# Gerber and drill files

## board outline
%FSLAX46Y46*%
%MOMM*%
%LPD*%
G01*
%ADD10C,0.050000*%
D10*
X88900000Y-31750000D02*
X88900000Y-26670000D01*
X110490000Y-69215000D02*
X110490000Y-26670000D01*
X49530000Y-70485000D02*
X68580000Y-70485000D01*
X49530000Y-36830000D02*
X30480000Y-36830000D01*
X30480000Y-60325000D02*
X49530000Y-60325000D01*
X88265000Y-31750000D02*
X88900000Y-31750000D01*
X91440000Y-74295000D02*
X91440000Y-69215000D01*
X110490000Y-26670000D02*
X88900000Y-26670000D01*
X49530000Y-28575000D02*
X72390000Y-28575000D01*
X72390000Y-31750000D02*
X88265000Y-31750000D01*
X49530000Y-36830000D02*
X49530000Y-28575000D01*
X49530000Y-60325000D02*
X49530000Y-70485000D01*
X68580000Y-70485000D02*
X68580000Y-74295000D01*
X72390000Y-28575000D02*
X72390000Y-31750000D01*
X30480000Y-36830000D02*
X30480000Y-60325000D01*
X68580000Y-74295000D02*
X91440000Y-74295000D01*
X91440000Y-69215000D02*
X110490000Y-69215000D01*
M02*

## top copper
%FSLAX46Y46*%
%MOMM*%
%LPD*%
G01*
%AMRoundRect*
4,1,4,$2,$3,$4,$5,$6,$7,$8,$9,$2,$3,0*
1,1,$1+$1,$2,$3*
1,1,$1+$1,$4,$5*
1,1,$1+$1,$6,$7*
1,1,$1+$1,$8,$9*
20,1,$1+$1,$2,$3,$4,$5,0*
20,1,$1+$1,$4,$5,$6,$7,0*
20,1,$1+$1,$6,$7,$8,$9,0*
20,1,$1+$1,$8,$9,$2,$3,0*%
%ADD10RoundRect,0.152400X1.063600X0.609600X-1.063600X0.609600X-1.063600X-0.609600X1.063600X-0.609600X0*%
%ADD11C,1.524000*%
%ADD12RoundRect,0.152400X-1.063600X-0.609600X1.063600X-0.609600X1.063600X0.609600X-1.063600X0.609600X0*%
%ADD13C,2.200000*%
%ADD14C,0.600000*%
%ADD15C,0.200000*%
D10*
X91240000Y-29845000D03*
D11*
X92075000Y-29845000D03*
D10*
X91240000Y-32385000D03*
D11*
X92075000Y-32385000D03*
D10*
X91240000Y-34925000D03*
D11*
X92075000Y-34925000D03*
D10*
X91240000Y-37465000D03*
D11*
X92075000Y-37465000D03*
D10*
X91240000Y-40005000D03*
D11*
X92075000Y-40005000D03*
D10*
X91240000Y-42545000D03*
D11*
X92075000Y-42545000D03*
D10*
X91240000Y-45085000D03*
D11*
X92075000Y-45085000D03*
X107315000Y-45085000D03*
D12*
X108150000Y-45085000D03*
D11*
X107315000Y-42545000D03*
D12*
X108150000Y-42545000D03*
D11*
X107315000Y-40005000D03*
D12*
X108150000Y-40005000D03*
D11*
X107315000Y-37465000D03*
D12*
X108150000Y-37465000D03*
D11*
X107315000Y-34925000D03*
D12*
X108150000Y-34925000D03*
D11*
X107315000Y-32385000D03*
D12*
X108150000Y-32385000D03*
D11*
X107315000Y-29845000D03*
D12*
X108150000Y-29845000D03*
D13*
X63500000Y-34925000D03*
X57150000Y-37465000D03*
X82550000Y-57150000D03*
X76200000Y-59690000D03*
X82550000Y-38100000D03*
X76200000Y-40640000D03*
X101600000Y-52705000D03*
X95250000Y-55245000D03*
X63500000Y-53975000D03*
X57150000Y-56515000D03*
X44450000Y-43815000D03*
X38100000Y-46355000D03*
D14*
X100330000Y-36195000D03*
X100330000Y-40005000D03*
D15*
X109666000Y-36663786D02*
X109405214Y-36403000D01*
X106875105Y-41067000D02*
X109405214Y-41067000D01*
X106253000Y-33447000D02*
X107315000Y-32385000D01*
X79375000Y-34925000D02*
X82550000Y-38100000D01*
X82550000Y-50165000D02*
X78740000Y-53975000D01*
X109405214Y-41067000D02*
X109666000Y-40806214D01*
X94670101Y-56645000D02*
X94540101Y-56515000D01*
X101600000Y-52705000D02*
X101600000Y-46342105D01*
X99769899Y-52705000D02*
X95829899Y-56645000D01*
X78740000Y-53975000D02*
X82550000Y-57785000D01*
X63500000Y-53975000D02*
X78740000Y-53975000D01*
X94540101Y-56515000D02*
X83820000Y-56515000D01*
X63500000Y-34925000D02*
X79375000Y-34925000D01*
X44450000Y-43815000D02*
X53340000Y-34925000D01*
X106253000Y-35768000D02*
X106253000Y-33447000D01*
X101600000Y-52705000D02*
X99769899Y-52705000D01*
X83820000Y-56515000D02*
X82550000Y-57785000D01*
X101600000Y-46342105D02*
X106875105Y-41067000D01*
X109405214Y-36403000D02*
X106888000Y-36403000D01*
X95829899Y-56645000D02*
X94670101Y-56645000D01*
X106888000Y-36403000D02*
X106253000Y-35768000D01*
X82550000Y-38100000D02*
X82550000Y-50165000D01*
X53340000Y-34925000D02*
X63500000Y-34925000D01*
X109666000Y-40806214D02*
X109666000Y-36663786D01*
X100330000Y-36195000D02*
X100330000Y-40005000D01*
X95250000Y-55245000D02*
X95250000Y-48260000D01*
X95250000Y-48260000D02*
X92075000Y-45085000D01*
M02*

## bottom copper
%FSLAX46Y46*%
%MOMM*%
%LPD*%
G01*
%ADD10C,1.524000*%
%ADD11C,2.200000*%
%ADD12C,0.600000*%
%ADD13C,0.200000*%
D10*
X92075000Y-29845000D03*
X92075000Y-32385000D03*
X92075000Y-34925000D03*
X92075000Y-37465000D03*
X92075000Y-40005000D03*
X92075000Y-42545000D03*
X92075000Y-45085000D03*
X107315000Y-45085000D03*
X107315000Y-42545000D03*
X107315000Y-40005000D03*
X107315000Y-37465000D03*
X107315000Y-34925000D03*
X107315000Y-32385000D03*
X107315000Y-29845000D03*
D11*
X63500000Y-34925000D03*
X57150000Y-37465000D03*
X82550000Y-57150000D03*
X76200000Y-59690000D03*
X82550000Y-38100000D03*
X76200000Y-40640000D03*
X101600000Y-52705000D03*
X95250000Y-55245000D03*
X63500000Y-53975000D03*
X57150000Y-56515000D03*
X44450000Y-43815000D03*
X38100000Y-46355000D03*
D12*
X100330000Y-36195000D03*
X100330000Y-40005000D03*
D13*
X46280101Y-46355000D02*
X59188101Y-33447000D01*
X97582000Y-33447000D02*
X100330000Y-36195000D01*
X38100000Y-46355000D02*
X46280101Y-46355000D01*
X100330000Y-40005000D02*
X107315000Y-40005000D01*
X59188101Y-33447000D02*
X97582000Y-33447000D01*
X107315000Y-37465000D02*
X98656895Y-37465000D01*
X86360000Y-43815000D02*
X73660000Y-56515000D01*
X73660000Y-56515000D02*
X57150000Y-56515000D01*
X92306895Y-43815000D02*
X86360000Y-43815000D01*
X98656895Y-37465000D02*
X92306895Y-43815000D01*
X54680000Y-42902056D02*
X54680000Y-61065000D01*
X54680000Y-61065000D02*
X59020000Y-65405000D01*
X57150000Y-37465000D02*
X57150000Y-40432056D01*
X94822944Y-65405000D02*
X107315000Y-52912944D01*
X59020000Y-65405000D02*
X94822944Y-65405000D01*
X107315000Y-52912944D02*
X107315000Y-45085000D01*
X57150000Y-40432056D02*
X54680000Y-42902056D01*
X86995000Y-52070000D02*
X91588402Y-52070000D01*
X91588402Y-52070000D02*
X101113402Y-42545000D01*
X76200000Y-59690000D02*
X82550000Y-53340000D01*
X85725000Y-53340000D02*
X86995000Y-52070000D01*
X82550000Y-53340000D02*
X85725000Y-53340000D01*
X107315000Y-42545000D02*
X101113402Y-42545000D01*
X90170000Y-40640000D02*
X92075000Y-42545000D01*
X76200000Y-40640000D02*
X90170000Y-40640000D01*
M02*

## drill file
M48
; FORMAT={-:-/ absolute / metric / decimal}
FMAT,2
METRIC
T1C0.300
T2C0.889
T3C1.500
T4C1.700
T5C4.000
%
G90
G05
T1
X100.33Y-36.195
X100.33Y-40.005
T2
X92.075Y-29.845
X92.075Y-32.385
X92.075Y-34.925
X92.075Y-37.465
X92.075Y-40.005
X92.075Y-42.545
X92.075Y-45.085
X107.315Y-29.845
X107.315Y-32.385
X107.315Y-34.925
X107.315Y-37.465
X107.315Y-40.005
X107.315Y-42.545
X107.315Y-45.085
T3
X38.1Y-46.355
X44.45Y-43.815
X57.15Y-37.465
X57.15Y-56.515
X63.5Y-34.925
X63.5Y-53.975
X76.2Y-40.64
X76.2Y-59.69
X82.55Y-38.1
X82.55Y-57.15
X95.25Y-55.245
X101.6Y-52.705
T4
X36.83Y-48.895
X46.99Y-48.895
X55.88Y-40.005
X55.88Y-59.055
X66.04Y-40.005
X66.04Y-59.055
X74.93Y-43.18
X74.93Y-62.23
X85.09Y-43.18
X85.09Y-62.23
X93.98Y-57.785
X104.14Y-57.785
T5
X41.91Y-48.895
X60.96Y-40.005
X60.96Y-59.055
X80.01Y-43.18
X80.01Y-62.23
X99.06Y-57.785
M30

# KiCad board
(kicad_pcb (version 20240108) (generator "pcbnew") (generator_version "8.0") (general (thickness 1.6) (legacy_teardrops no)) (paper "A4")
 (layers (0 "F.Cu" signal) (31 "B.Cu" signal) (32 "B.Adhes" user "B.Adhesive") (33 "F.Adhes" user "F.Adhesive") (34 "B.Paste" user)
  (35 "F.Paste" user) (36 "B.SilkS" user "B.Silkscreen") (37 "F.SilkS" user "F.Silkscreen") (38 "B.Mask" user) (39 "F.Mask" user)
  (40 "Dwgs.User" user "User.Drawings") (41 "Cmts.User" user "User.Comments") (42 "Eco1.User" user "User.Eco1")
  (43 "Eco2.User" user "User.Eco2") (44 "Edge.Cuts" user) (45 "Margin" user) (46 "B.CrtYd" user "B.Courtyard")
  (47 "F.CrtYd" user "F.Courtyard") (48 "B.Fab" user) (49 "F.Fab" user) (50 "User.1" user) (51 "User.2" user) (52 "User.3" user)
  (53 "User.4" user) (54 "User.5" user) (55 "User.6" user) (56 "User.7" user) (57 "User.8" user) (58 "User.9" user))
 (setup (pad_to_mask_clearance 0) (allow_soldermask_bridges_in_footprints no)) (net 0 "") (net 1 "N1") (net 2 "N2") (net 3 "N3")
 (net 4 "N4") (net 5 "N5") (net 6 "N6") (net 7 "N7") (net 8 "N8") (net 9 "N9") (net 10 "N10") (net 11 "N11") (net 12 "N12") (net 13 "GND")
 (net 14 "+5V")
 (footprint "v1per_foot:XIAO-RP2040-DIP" (layer "F.Cu") (at 99.695 37.465)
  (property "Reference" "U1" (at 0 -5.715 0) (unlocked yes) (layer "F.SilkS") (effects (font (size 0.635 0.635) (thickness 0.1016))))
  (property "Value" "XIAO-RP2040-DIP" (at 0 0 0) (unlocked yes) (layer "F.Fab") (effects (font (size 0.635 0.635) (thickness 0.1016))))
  (pad "1" smd roundrect (at -8.455 -7.62 180) (size 2.432 1.524) (layers "F.Cu" "F.Mask") (roundrect_rratio 0.1) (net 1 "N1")
   (thermal_bridge_angle 45))
  (pad "1" thru_hole circle (at -7.62 -7.62 180) (size 1.524 1.524) (drill 0.889) (layers "*.Cu" "*.Mask") (remove_unused_layers no)
   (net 1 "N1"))
  (pad "2" smd roundrect (at -8.455 -5.08 180) (size 2.432 1.524) (layers "F.Cu" "F.Mask") (roundrect_rratio 0.1) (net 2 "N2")
   (thermal_bridge_angle 45))
  (pad "2" thru_hole circle (at -7.62 -5.08 180) (size 1.524 1.524) (drill 0.889) (layers "*.Cu" "*.Mask") (remove_unused_layers no)
   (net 2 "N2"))
  (pad "3" smd roundrect (at -8.455 -2.54 180) (size 2.432 1.524) (layers "F.Cu" "F.Mask") (roundrect_rratio 0.1) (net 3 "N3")
   (thermal_bridge_angle 45))
  (pad "3" thru_hole circle (at -7.62 -2.54 180) (size 1.524 1.524) (drill 0.889) (layers "*.Cu" "*.Mask") (remove_unused_layers no)
   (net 3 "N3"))
  (pad "4" smd roundrect (at -8.455 0 180) (size 2.432 1.524) (layers "F.Cu" "F.Mask") (roundrect_rratio 0.1) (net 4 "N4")
   (thermal_bridge_angle 45))
  (pad "4" thru_hole circle (at -7.62 0 180) (size 1.524 1.524) (drill 0.889) (layers "*.Cu" "*.Mask") (remove_unused_layers no)
   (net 4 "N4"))
  (pad "5" smd roundrect (at -8.455 2.54 180) (size 2.432 1.524) (layers "F.Cu" "F.Mask") (roundrect_rratio 0.1) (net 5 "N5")
   (thermal_bridge_angle 45))
  (pad "5" thru_hole circle (at -7.62 2.54 180) (size 1.524 1.524) (drill 0.889) (layers "*.Cu" "*.Mask") (remove_unused_layers no)
   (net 5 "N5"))
  (pad "6" smd roundrect (at -8.455 5.08 180) (size 2.432 1.524) (layers "F.Cu" "F.Mask") (roundrect_rratio 0.1) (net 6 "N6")
   (thermal_bridge_angle 45))
  (pad "6" thru_hole circle (at -7.62 5.08 180) (size 1.524 1.524) (drill 0.889) (layers "*.Cu" "*.Mask") (remove_unused_layers no)
   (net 6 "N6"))
  (pad "7" smd roundrect (at -8.455 7.62 180) (size 2.432 1.524) (layers "F.Cu" "F.Mask") (roundrect_rratio 0.1) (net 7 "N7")
   (thermal_bridge_angle 45))
  (pad "7" thru_hole circle (at -7.62 7.62 180) (size 1.524 1.524) (drill 0.889) (layers "*.Cu" "*.Mask") (remove_unused_layers no)
   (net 7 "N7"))
  (pad "8" thru_hole circle (at 7.62 7.62) (size 1.524 1.524) (drill 0.889) (layers "*.Cu" "*.Mask") (remove_unused_layers no) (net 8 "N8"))
  (pad "8" smd roundrect (at 8.455 7.62) (size 2.432 1.524) (layers "F.Cu" "F.Mask") (roundrect_rratio 0.1) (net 8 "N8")
   (thermal_bridge_angle 45))
  (pad "9" thru_hole circle (at 7.62 5.08) (size 1.524 1.524) (drill 0.889) (layers "*.Cu" "*.Mask") (remove_unused_layers no) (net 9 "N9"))
  (pad "9" smd roundrect (at 8.455 5.08) (size 2.432 1.524) (layers "F.Cu" "F.Mask") (roundrect_rratio 0.1) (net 9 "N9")
   (thermal_bridge_angle 45))
  (pad "10" thru_hole circle (at 7.62 2.54) (size 1.524 1.524) (drill 0.889) (layers "*.Cu" "*.Mask") (remove_unused_layers no)
   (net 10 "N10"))
  (pad "10" smd roundrect (at 8.455 2.54) (size 2.432 1.524) (layers "F.Cu" "F.Mask") (roundrect_rratio 0.1) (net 10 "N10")
   (thermal_bridge_angle 45))
  (pad "11" thru_hole circle (at 7.62 0) (size 1.524 1.524) (drill 0.889) (layers "*.Cu" "*.Mask") (remove_unused_layers no) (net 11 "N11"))
  (pad "11" smd roundrect (at 8.455 0) (size 2.432 1.524) (layers "F.Cu" "F.Mask") (roundrect_rratio 0.1) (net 11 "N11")
   (thermal_bridge_angle 45))
  (pad "12" thru_hole circle (at 7.62 -2.54) (size 1.524 1.524) (drill 0.889) (layers "*.Cu" "*.Mask") (remove_unused_layers no)
   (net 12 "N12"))
  (pad "12" smd roundrect (at 8.455 -2.54) (size 2.432 1.524) (layers "F.Cu" "F.Mask") (roundrect_rratio 0.1) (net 12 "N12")
   (thermal_bridge_angle 45))
  (pad "13" thru_hole circle (at 7.62 -5.08) (size 1.524 1.524) (drill 0.889) (layers "*.Cu" "*.Mask") (remove_unused_layers no)
   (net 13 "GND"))
  (pad "13" smd roundrect (at 8.455 -5.08) (size 2.432 1.524) (layers "F.Cu" "F.Mask") (roundrect_rratio 0.1) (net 13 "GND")
   (thermal_bridge_angle 45))
  (pad "14" thru_hole circle (at 7.62 -7.62) (size 1.524 1.524) (drill 0.889) (layers "*.Cu" "*.Mask") (remove_unused_layers no)
   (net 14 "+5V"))
  (pad "14" smd roundrect (at 8.455 -7.62) (size 2.432 1.524) (layers "F.Cu" "F.Mask") (roundrect_rratio 0.1) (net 14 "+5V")
   (thermal_bridge_angle 45)))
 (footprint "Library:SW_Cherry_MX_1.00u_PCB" (layer "F.Cu") (at 63.5 34.925)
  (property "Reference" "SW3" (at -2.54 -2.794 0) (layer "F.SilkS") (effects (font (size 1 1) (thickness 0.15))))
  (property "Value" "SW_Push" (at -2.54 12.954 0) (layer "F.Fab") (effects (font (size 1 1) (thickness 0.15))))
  (pad "" np_thru_hole circle (at -7.62 5.08) (size 1.7 1.7) (drill 1.7) (layers "*.Cu" "*.Mask"))
  (pad "" np_thru_hole circle (at -2.54 5.08) (size 4 4) (drill 4) (layers "*.Cu" "*.Mask"))
  (pad "" np_thru_hole circle (at 2.54 5.08) (size 1.7 1.7) (drill 1.7) (layers "*.Cu" "*.Mask"))
  (pad "1" thru_hole circle (at 0 0) (size 2.2 2.2) (drill 1.5) (layers "*.Cu" "*.Mask") (remove_unused_layers no) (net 13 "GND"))
  (pad "2" thru_hole circle (at -6.35 2.54) (size 2.2 2.2) (drill 1.5) (layers "*.Cu" "*.Mask") (remove_unused_layers no) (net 8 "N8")))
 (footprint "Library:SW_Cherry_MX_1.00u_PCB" (layer "F.Cu") (at 82.55 57.15)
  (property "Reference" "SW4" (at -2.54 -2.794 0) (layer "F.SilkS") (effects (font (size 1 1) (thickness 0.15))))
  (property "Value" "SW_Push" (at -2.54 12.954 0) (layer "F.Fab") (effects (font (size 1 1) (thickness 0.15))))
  (pad "" np_thru_hole circle (at -7.62 5.08) (size 1.7 1.7) (drill 1.7) (layers "*.Cu" "*.Mask"))
  (pad "" np_thru_hole circle (at -2.54 5.08) (size 4 4) (drill 4) (layers "*.Cu" "*.Mask"))
  (pad "" np_thru_hole circle (at 2.54 5.08) (size 1.7 1.7) (drill 1.7) (layers "*.Cu" "*.Mask"))
  (pad "1" thru_hole circle (at 0 0) (size 2.2 2.2) (drill 1.5) (layers "*.Cu" "*.Mask") (remove_unused_layers no) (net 13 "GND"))
  (pad "2" thru_hole circle (at -6.35 2.54) (size 2.2 2.2) (drill 1.5) (layers "*.Cu" "*.Mask") (remove_unused_layers no) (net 9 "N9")))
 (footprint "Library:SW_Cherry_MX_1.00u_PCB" (layer "F.Cu") (at 82.55 38.1)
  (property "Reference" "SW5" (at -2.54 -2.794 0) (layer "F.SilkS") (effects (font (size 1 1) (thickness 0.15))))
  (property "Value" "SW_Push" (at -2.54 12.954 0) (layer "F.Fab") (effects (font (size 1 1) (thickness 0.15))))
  (pad "" np_thru_hole circle (at -7.62 5.08) (size 1.7 1.7) (drill 1.7) (layers "*.Cu" "*.Mask"))
  (pad "" np_thru_hole circle (at -2.54 5.08) (size 4 4) (drill 4) (layers "*.Cu" "*.Mask"))
  (pad "" np_thru_hole circle (at 2.54 5.08) (size 1.7 1.7) (drill 1.7) (layers "*.Cu" "*.Mask"))
  (pad "1" thru_hole circle (at 0 0) (size 2.2 2.2) (drill 1.5) (layers "*.Cu" "*.Mask") (remove_unused_layers no) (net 13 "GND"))
  (pad "2" thru_hole circle (at -6.35 2.54) (size 2.2 2.2) (drill 1.5) (layers "*.Cu" "*.Mask") (remove_unused_layers no) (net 6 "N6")))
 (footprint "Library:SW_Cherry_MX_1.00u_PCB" (layer "F.Cu") (at 101.6 52.705)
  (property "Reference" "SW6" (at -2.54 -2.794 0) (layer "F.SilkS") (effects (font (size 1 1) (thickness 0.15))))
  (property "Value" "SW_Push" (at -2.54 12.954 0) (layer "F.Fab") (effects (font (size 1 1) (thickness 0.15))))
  (pad "" np_thru_hole circle (at -7.62 5.08) (size 1.7 1.7) (drill 1.7) (layers "*.Cu" "*.Mask"))
  (pad "" np_thru_hole circle (at -2.54 5.08) (size 4 4) (drill 4) (layers "*.Cu" "*.Mask"))
  (pad "" np_thru_hole circle (at 2.54 5.08) (size 1.7 1.7) (drill 1.7) (layers "*.Cu" "*.Mask"))
  (pad "1" thru_hole circle (at 0 0) (size 2.2 2.2) (drill 1.5) (layers "*.Cu" "*.Mask") (remove_unused_layers no) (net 13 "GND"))
  (pad "2" thru_hole circle (at -6.35 2.54) (size 2.2 2.2) (drill 1.5) (layers "*.Cu" "*.Mask") (remove_unused_layers no) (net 7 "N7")))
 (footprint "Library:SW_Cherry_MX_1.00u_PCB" (layer "F.Cu") (at 63.5 53.975)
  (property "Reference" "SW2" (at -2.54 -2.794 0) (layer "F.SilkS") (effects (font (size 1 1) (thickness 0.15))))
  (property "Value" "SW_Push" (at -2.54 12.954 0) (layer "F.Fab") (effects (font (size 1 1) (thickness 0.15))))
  (pad "" np_thru_hole circle (at -7.62 5.08) (size 1.7 1.7) (drill 1.7) (layers "*.Cu" "*.Mask"))
  (pad "" np_thru_hole circle (at -2.54 5.08) (size 4 4) (drill 4) (layers "*.Cu" "*.Mask"))
  (pad "" np_thru_hole circle (at 2.54 5.08) (size 1.7 1.7) (drill 1.7) (layers "*.Cu" "*.Mask"))
  (pad "1" thru_hole circle (at 0 0) (size 2.2 2.2) (drill 1.5) (layers "*.Cu" "*.Mask") (remove_unused_layers no) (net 13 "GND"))
  (pad "2" thru_hole circle (at -6.35 2.54) (size 2.2 2.2) (drill 1.5) (layers "*.Cu" "*.Mask") (remove_unused_layers no) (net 11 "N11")))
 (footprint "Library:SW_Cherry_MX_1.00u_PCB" (layer "F.Cu") (at 44.45 43.815)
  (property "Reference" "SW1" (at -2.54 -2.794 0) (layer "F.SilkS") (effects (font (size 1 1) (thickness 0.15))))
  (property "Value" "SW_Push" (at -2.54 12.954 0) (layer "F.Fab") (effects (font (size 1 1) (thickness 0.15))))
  (pad "" np_thru_hole circle (at -7.62 5.08) (size 1.7 1.7) (drill 1.7) (layers "*.Cu" "*.Mask"))
  (pad "" np_thru_hole circle (at -2.54 5.08) (size 4 4) (drill 4) (layers "*.Cu" "*.Mask"))
  (pad "" np_thru_hole circle (at 2.54 5.08) (size 1.7 1.7) (drill 1.7) (layers "*.Cu" "*.Mask"))
  (pad "1" thru_hole circle (at 0 0) (size 2.2 2.2) (drill 1.5) (layers "*.Cu" "*.Mask") (remove_unused_layers no) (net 13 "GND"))
  (pad "2" thru_hole circle (at -6.35 2.54) (size 2.2 2.2) (drill 1.5) (layers "*.Cu" "*.Mask") (remove_unused_layers no) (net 10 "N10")))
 (gr_line (start 88.9 31.75) (end 88.9 26.67) (stroke (width 0.05) (type default)) (layer "Edge.Cuts"))
 (gr_line (start 110.49 69.215) (end 110.49 26.67) (stroke (width 0.05) (type default)) (layer "Edge.Cuts"))
 (gr_line (start 49.53 70.485) (end 68.58 70.485) (stroke (width 0.05) (type default)) (layer "Edge.Cuts"))
 (gr_line (start 49.53 36.83) (end 30.48 36.83) (stroke (width 0.05) (type default)) (layer "Edge.Cuts"))
 (gr_line (start 30.48 60.325) (end 49.53 60.325) (stroke (width 0.05) (type default)) (layer "Edge.Cuts"))
 (gr_line (start 88.265 31.75) (end 88.9 31.75) (stroke (width 0.05) (type default)) (layer "Edge.Cuts"))
 (gr_line (start 91.44 74.295) (end 91.44 69.215) (stroke (width 0.05) (type default)) (layer "Edge.Cuts"))
 (gr_line (start 110.49 26.67) (end 88.9 26.67) (stroke (width 0.05) (type default)) (layer "Edge.Cuts"))
 (gr_line (start 49.53 28.575) (end 72.39 28.575) (stroke (width 0.05) (type default)) (layer "Edge.Cuts"))
 (gr_line (start 72.39 31.75) (end 88.265 31.75) (stroke (width 0.05) (type default)) (layer "Edge.Cuts"))
 (gr_line (start 49.53 36.83) (end 49.53 28.575) (stroke (width 0.05) (type default)) (layer "Edge.Cuts"))
 (gr_line (start 49.53 60.325) (end 49.53 70.485) (stroke (width 0.05) (type default)) (layer "Edge.Cuts"))
 (gr_line (start 68.58 70.485) (end 68.58 74.295) (stroke (width 0.05) (type default)) (layer "Edge.Cuts"))
 (gr_line (start 72.39 28.575) (end 72.39 31.75) (stroke (width 0.05) (type default)) (layer "Edge.Cuts"))
 (gr_line (start 30.48 36.83) (end 30.48 60.325) (stroke (width 0.05) (type default)) (layer "Edge.Cuts"))
 (gr_line (start 68.58 74.295) (end 91.44 74.295) (stroke (width 0.05) (type default)) (layer "Edge.Cuts"))
 (gr_line (start 91.44 69.215) (end 110.49 69.215) (stroke (width 0.05) (type default)) (layer "Edge.Cuts"))
 (segment (start 109.666 36.663786) (end 109.405214 36.403) (width 0.2) (layer "F.Cu") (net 13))
 (segment (start 106.875105 41.067) (end 109.405214 41.067) (width 0.2) (layer "F.Cu") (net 13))
 (segment (start 106.253 33.447) (end 107.315 32.385) (width 0.2) (layer "F.Cu") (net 13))
 (segment (start 79.375 34.925) (end 82.55 38.1) (width 0.2) (layer "F.Cu") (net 13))
 (segment (start 82.55 50.165) (end 78.74 53.975) (width 0.2) (layer "F.Cu") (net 13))
 (segment (start 109.405214 41.067) (end 109.666 40.806214) (width 0.2) (layer "F.Cu") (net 13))
 (segment (start 94.670101 56.645) (end 94.540101 56.515) (width 0.2) (layer "F.Cu") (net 13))
 (segment (start 101.6 52.705) (end 101.6 46.342105) (width 0.2) (layer "F.Cu") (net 13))
 (segment (start 99.769899 52.705) (end 95.829899 56.645) (width 0.2) (layer "F.Cu") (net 13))
 (segment (start 78.74 53.975) (end 82.55 57.785) (width 0.2) (layer "F.Cu") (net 13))
 (segment (start 63.5 53.975) (end 78.74 53.975) (width 0.2) (layer "F.Cu") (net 13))
 (segment (start 94.540101 56.515) (end 83.82 56.515) (width 0.2) (layer "F.Cu") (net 13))
 (segment (start 63.5 34.925) (end 79.375 34.925) (width 0.2) (layer "F.Cu") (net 13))
 (segment (start 44.45 43.815) (end 53.34 34.925) (width 0.2) (layer "F.Cu") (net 13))
 (segment (start 106.253 35.768) (end 106.253 33.447) (width 0.2) (layer "F.Cu") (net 13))
 (segment (start 101.6 52.705) (end 99.769899 52.705) (width 0.2) (layer "F.Cu") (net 13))
 (segment (start 83.82 56.515) (end 82.55 57.785) (width 0.2) (layer "F.Cu") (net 13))
 (segment (start 101.6 46.342105) (end 106.875105 41.067) (width 0.2) (layer "F.Cu") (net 13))
 (segment (start 109.405214 36.403) (end 106.888 36.403) (width 0.2) (layer "F.Cu") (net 13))
 (segment (start 95.829899 56.645) (end 94.670101 56.645) (width 0.2) (layer "F.Cu") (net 13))
 (segment (start 106.888 36.403) (end 106.253 35.768) (width 0.2) (layer "F.Cu") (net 13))
 (segment (start 82.55 38.1) (end 82.55 50.165) (width 0.2) (layer "F.Cu") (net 13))
 (segment (start 53.34 34.925) (end 63.5 34.925) (width 0.2) (layer "F.Cu") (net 13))
 (segment (start 109.666 40.806214) (end 109.666 36.663786) (width 0.2) (layer "F.Cu") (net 13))
 (segment (start 100.33 36.195) (end 100.33 40.005) (width 0.2) (layer "F.Cu") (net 10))
 (via (at 100.33 36.195) (size 0.6) (drill 0.3) (layers "F.Cu" "B.Cu") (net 10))
 (via (at 100.33 40.005) (size 0.6) (drill 0.3) (layers "F.Cu" "B.Cu") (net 10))
 (segment (start 46.280101 46.355) (end 59.188101 33.447) (width 0.2) (layer "B.Cu") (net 10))
 (segment (start 97.582 33.447) (end 100.33 36.195) (width 0.2) (layer "B.Cu") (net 10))
 (segment (start 38.1 46.355) (end 46.280101 46.355) (width 0.2) (layer "B.Cu") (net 10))
 (segment (start 100.33 40.005) (end 107.315 40.005) (width 0.2) (layer "B.Cu") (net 10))
 (segment (start 59.188101 33.447) (end 97.582 33.447) (width 0.2) (layer "B.Cu") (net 10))
 (segment (start 107.315 37.465) (end 98.656895 37.465) (width 0.2) (layer "B.Cu") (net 11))
 (segment (start 86.36 43.815) (end 73.66 56.515) (width 0.2) (layer "B.Cu") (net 11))
 (segment (start 73.66 56.515) (end 57.15 56.515) (width 0.2) (layer "B.Cu") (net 11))
 (segment (start 92.306895 43.815) (end 86.36 43.815) (width 0.2) (layer "B.Cu") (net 11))
 (segment (start 98.656895 37.465) (end 92.306895 43.815) (width 0.2) (layer "B.Cu") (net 11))
 (segment (start 54.68 42.902056) (end 54.68 61.065) (width 0.2) (layer "B.Cu") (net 8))
 (segment (start 54.68 61.065) (end 59.02 65.405) (width 0.2) (layer "B.Cu") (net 8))
 (segment (start 57.15 37.465) (end 57.15 40.432056) (width 0.2) (layer "B.Cu") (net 8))
 (segment (start 94.822944 65.405) (end 107.315 52.912944) (width 0.2) (layer "B.Cu") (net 8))
 (segment (start 59.02 65.405) (end 94.822944 65.405) (width 0.2) (layer "B.Cu") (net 8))
 (segment (start 107.315 52.912944) (end 107.315 45.085) (width 0.2) (layer "B.Cu") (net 8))
 (segment (start 57.15 40.432056) (end 54.68 42.902056) (width 0.2) (layer "B.Cu") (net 8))
 (segment (start 86.995 52.07) (end 91.588402 52.07) (width 0.2) (layer "B.Cu") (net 9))
 (segment (start 91.588402 52.07) (end 101.113402 42.545) (width 0.2) (layer "B.Cu") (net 9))
 (segment (start 76.2 59.69) (end 82.55 53.34) (width 0.2) (layer "B.Cu") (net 9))
 (segment (start 85.725 53.34) (end 86.995 52.07) (width 0.2) (layer "B.Cu") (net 9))
 (segment (start 82.55 53.34) (end 85.725 53.34) (width 0.2) (layer "B.Cu") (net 9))
 (segment (start 107.315 42.545) (end 101.113402 42.545) (width 0.2) (layer "B.Cu") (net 9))
 (segment (start 90.17 40.64) (end 92.075 42.545) (width 0.2) (layer "B.Cu") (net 6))
 (segment (start 76.2 40.64) (end 90.17 40.64) (width 0.2) (layer "B.Cu") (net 6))
 (segment (start 95.25 55.245) (end 95.25 48.26) (width 0.2) (layer "F.Cu") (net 7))
 (segment (start 95.25 48.26) (end 92.075 45.085) (width 0.2) (layer "F.Cu") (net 7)))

